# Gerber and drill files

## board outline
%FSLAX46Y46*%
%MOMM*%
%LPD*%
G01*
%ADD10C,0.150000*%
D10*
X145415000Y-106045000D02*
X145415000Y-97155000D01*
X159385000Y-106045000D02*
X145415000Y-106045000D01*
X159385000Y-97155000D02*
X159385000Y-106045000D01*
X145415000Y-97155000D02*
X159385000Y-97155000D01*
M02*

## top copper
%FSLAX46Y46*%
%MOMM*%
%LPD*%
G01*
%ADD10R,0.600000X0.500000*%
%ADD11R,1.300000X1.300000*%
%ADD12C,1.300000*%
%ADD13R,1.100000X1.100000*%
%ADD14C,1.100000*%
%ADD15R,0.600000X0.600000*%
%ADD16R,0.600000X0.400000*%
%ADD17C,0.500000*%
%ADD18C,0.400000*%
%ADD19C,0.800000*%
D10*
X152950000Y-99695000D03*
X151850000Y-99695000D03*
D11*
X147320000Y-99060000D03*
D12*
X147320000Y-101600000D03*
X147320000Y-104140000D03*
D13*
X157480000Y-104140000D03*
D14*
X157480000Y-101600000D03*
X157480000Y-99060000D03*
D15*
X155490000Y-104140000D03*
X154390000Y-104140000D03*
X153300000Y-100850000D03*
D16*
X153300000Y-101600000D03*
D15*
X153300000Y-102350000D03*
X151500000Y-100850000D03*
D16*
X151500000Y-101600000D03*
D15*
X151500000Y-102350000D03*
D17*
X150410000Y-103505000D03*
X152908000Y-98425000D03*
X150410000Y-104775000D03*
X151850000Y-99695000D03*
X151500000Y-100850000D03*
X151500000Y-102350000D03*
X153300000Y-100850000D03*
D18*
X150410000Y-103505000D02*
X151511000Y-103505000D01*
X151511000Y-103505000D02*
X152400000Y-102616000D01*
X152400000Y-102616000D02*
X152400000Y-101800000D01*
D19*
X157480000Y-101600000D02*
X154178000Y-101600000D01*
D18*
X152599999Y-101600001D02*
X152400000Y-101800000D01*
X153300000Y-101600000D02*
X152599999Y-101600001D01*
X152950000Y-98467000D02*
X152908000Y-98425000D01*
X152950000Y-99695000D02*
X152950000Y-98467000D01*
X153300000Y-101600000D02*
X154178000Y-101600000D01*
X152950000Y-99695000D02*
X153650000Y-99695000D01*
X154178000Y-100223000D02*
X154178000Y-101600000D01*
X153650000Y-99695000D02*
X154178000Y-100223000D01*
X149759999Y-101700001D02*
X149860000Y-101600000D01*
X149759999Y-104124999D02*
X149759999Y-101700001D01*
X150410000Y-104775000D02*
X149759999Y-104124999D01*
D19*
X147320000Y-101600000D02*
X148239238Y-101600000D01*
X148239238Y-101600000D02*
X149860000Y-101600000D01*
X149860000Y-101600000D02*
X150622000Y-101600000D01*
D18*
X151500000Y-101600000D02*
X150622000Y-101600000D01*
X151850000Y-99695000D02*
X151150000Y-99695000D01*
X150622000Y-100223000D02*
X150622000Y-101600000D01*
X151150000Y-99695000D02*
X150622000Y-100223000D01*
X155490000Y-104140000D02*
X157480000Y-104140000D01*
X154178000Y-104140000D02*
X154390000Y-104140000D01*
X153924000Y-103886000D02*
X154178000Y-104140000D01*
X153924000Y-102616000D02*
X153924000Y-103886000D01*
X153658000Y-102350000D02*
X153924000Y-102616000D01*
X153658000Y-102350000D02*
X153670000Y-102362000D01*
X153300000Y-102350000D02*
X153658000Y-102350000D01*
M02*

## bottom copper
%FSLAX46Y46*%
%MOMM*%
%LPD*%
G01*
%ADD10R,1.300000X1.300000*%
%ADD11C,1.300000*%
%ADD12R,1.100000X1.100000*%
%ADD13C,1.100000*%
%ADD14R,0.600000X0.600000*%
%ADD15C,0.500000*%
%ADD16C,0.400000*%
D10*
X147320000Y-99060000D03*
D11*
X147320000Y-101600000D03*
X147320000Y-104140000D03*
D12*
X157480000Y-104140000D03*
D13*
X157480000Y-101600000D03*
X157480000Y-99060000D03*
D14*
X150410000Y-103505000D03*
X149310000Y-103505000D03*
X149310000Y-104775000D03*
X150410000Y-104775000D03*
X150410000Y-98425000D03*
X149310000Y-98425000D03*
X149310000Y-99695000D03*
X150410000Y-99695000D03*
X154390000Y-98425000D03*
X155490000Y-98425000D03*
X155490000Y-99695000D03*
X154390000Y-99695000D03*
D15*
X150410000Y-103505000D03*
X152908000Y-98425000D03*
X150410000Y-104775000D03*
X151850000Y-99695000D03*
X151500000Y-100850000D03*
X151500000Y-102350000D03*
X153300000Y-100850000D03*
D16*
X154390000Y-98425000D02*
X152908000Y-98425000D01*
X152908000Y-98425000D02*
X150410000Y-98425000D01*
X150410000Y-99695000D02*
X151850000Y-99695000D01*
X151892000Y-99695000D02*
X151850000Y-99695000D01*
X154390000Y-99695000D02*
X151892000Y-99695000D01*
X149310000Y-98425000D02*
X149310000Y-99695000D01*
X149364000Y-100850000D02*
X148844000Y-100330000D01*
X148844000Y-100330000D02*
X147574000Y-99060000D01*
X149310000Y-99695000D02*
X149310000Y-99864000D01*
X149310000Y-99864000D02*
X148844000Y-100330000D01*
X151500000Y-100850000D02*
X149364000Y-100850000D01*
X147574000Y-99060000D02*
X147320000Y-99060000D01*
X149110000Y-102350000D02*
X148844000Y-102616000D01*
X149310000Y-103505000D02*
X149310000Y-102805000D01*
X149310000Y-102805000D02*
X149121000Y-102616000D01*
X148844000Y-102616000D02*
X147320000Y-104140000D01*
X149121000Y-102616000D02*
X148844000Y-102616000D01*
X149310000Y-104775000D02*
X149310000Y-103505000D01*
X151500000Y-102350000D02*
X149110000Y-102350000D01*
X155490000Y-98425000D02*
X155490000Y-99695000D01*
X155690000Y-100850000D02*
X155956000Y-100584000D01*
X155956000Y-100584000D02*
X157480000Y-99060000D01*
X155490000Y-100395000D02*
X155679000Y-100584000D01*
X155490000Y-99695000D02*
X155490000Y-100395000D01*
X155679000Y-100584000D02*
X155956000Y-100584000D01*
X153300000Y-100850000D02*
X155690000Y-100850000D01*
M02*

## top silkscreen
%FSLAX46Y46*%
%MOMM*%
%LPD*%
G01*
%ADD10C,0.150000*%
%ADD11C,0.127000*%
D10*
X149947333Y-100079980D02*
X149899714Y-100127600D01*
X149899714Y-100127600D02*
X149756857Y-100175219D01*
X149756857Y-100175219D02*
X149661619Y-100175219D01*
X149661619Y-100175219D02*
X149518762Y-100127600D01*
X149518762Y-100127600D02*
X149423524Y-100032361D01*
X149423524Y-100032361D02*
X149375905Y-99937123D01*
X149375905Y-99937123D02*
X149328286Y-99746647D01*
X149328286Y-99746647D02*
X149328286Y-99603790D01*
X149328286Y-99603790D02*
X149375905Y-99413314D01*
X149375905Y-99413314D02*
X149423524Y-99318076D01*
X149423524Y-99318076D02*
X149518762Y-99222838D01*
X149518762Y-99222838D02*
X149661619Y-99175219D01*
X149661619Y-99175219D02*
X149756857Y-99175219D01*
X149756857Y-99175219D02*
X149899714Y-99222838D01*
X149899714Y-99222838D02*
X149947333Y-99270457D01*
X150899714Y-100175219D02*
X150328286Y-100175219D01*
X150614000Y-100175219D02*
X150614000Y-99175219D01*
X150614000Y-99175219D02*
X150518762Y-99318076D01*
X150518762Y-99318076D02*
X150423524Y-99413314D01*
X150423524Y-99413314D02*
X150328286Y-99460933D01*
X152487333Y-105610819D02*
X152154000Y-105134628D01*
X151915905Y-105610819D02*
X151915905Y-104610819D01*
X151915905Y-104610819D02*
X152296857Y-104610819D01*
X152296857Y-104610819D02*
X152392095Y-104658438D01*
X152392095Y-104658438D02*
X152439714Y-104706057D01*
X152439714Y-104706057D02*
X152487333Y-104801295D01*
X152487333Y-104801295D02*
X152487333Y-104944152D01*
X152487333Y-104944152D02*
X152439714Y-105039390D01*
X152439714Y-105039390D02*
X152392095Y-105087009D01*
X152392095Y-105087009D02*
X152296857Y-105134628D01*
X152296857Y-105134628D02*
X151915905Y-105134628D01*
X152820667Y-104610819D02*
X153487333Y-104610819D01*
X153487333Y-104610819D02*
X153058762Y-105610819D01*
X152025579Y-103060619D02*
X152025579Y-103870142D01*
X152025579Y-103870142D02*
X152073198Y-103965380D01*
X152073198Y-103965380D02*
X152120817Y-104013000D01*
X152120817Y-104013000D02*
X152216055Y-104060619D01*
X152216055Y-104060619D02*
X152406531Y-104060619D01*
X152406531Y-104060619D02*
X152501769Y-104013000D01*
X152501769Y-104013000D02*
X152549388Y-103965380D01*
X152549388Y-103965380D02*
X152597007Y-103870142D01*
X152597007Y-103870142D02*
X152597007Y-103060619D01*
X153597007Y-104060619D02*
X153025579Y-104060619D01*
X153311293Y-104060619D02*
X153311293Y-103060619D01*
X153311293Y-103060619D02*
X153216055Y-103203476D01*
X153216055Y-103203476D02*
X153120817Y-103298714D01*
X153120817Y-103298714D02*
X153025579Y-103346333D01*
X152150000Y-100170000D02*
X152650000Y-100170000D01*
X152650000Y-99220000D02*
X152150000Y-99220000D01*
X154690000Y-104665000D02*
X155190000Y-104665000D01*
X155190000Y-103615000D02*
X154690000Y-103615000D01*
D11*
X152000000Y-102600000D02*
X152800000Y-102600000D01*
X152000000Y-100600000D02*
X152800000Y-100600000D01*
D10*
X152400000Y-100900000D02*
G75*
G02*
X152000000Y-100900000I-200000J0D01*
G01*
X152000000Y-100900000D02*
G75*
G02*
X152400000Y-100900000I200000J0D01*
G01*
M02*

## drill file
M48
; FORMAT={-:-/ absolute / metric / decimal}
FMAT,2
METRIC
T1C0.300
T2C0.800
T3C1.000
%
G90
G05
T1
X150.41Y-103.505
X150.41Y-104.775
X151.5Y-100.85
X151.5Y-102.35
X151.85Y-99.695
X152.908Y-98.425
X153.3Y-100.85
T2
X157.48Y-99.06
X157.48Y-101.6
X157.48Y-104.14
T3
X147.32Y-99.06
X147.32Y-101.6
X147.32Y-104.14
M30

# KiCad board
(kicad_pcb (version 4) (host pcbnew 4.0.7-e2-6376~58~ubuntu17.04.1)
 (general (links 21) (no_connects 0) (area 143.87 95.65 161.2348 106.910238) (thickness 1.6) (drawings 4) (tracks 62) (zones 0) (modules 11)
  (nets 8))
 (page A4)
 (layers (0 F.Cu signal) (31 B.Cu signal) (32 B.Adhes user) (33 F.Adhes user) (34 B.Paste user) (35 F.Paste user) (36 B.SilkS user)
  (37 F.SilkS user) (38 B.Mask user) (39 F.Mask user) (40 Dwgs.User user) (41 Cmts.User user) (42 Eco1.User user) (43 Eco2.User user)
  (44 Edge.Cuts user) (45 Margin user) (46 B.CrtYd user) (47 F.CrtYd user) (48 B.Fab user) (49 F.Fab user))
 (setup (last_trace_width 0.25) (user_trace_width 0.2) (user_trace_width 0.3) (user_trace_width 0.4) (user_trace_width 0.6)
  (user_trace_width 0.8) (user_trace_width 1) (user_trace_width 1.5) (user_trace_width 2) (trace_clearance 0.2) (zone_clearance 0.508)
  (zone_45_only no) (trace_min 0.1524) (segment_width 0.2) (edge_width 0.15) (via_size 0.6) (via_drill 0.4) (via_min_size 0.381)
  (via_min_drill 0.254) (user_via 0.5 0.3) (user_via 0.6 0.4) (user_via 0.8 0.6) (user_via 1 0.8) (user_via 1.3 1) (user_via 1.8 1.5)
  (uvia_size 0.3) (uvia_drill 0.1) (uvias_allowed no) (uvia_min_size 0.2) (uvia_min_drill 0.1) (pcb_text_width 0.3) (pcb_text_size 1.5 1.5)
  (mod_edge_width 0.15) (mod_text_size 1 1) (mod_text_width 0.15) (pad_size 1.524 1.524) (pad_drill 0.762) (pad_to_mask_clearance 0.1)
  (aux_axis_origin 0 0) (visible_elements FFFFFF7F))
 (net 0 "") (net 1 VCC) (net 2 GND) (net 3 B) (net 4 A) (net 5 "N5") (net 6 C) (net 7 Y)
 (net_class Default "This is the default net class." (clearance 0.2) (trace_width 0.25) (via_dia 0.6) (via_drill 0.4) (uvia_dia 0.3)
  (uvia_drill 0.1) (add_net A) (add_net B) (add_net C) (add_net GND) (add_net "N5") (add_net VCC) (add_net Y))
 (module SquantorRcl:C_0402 (layer F.Cu) (at 152.4 99.695 180)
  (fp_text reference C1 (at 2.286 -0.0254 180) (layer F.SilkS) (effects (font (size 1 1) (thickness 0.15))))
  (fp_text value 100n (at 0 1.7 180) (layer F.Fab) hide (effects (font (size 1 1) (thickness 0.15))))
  (fp_line (start 0.25 -0.475) (end -0.25 -0.475) (layer F.SilkS) (width 0.15))
  (fp_line (start -0.25 0.475) (end 0.25 0.475) (layer F.SilkS) (width 0.15))
  (pad 1 smd rect (at -0.55 0 180) (size 0.6 0.5) (layers F.Cu F.Paste F.Mask) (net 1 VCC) (solder_mask_margin 0.1))
  (pad 2 smd rect (at 0.55 0 180) (size 0.6 0.5) (layers F.Cu F.Paste F.Mask) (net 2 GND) (solder_mask_margin 0.1)))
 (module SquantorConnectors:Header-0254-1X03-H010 (layer B.Cu) (at 147.32 101.6 270)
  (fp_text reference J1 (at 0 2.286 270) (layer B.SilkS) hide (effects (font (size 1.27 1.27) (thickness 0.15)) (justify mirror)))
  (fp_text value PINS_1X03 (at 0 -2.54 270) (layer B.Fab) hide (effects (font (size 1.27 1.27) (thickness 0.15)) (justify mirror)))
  (pad 1 thru_hole rect (at -2.54 0 90) (size 1.3 1.3) (drill 1) (layers *.Cu *.Mask) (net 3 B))
  (pad 2 thru_hole circle (at 0 0 90) (size 1.3 1.3) (drill 1) (layers *.Cu *.Mask) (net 2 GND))
  (pad 3 thru_hole circle (at 2.54 0 90) (size 1.3 1.3) (drill 1) (layers *.Cu *.Mask) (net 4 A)))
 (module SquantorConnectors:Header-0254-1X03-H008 (layer B.Cu) (at 157.48 101.6 90)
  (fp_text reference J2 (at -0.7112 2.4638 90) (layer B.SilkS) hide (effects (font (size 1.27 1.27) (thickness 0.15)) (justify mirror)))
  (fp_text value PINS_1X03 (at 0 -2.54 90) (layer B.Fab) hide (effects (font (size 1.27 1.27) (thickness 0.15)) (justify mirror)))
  (pad 1 thru_hole rect (at -2.54 0 270) (size 1.1 1.1) (drill 0.8) (layers *.Cu *.Mask) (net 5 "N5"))
  (pad 2 thru_hole circle (at 0 0 270) (size 1.1 1.1) (drill 0.8) (layers *.Cu *.Mask) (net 1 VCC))
  (pad 3 thru_hole circle (at 2.54 0 270) (size 1.1 1.1) (drill 0.8) (layers *.Cu *.Mask) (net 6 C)))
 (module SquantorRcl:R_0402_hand (layer B.Cu) (at 149.86 103.505 180)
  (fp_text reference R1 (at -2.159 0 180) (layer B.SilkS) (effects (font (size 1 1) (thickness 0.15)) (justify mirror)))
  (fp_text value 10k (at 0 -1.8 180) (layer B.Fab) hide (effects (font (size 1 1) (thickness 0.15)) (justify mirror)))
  (pad 1 smd rect (at -0.55 0 180) (size 0.6 0.6) (layers B.Cu B.Paste B.Mask) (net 1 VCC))
  (pad 2 smd rect (at 0.55 0 180) (size 0.6 0.6) (layers B.Cu B.Paste B.Mask) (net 4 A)))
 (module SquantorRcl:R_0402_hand (layer B.Cu) (at 149.86 104.775)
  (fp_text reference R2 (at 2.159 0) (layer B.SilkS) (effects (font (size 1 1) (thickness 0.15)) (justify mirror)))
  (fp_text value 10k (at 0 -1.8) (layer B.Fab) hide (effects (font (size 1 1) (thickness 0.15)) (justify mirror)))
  (pad 1 smd rect (at -0.55 0) (size 0.6 0.6) (layers B.Cu B.Paste B.Mask) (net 4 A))
  (pad 2 smd rect (at 0.55 0) (size 0.6 0.6) (layers B.Cu B.Paste B.Mask) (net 2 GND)))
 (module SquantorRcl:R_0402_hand (layer B.Cu) (at 149.86 98.425 180)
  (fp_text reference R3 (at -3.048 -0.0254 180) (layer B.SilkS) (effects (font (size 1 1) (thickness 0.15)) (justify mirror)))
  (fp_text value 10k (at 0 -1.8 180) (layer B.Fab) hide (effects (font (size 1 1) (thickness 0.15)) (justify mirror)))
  (pad 1 smd rect (at -0.55 0 180) (size 0.6 0.6) (layers B.Cu B.Paste B.Mask) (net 1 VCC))
  (pad 2 smd rect (at 0.55 0 180) (size 0.6 0.6) (layers B.Cu B.Paste B.Mask) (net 3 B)))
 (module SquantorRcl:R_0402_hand (layer B.Cu) (at 149.86 99.695)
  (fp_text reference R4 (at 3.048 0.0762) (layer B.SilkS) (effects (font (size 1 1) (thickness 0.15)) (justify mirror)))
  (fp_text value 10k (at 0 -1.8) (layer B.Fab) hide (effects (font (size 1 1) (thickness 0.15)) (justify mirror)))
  (pad 1 smd rect (at -0.55 0) (size 0.6 0.6) (layers B.Cu B.Paste B.Mask) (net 3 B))
  (pad 2 smd rect (at 0.55 0) (size 0.6 0.6) (layers B.Cu B.Paste B.Mask) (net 2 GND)))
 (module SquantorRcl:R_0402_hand (layer B.Cu) (at 154.94 98.425)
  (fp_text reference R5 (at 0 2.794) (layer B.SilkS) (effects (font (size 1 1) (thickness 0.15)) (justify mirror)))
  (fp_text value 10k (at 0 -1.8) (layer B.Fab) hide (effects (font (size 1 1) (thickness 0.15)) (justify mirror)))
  (pad 1 smd rect (at -0.55 0) (size 0.6 0.6) (layers B.Cu B.Paste B.Mask) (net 1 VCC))
  (pad 2 smd rect (at 0.55 0) (size 0.6 0.6) (layers B.Cu B.Paste B.Mask) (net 6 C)))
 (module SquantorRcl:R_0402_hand (layer B.Cu) (at 154.94 99.695 180)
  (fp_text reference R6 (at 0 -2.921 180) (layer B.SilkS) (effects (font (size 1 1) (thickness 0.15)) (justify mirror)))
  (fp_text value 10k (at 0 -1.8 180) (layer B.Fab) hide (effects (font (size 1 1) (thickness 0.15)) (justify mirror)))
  (pad 1 smd rect (at -0.55 0 180) (size 0.6 0.6) (layers B.Cu B.Paste B.Mask) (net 6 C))
  (pad 2 smd rect (at 0.55 0 180) (size 0.6 0.6) (layers B.Cu B.Paste B.Mask) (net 2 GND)))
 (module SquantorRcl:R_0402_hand (layer F.Cu) (at 154.94 104.14 180)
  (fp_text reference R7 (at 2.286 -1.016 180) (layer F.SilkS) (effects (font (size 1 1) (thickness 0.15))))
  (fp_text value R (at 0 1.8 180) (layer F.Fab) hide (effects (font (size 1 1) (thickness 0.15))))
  (fp_line (start 0.25 -0.525) (end -0.25 -0.525) (layer F.SilkS) (width 0.15))
  (fp_line (start -0.25 0.525) (end 0.25 0.525) (layer F.SilkS) (width 0.15))
  (pad 1 smd rect (at -0.55 0 180) (size 0.6 0.6) (layers F.Cu F.Paste F.Mask) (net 5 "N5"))
  (pad 2 smd rect (at 0.55 0 180) (size 0.6 0.6) (layers F.Cu F.Paste F.Mask) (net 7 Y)))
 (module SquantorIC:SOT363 (layer F.Cu) (at 152.4 101.6 270)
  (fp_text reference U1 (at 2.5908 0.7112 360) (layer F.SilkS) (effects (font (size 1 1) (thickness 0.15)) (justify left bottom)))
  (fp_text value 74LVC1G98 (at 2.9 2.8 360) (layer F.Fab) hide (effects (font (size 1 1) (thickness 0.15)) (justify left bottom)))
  (fp_line (start 1 0.4) (end 1 -0.4) (layer F.SilkS) (width 0.127))
  (fp_line (start -1 0.4) (end -1 -0.4) (layer F.SilkS) (width 0.127))
  (fp_circle (center -0.7 0.2) (end -0.5 0.2) (layer F.SilkS) (width 0.15))
  (pad 6 smd rect (at -0.75 -0.9 270) (size 0.6 0.6) (layers F.Cu F.Paste F.Mask) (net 6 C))
  (pad 5 smd rect (at 0 -0.9 270) (size 0.4 0.6) (layers F.Cu F.Paste F.Mask) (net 1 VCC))
  (pad 4 smd rect (at 0.75 -0.9 270) (size 0.6 0.6) (layers F.Cu F.Paste F.Mask) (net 7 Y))
  (pad 1 smd rect (at -0.75 0.9 270) (size 0.6 0.6) (layers F.Cu F.Paste F.Mask) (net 3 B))
  (pad 2 smd rect (at 0 0.9 270) (size 0.4 0.6) (layers F.Cu F.Paste F.Mask) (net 2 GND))
  (pad 3 smd rect (at 0.75 0.9 270) (size 0.6 0.6) (layers F.Cu F.Paste F.Mask) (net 4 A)))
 (gr_line (start 145.415 106.045) (end 145.415 97.155) (angle 90) (layer Edge.Cuts) (width 0.15))
 (gr_line (start 159.385 106.045) (end 145.415 106.045) (angle 90) (layer Edge.Cuts) (width 0.15))
 (gr_line (start 159.385 97.155) (end 159.385 106.045) (angle 90) (layer Edge.Cuts) (width 0.15))
 (gr_line (start 145.415 97.155) (end 159.385 97.155) (angle 90) (layer Edge.Cuts) (width 0.15))
 (segment (start 150.41 103.505) (end 151.511 103.505) (width 0.4) (layer F.Cu) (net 1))
 (segment (start 151.511 103.505) (end 152.4 102.616) (width 0.4) (layer F.Cu) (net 1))
 (segment (start 152.4 102.616) (end 152.4 101.8) (width 0.4) (layer F.Cu) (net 1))
 (via (at 150.41 103.505) (size 0.5) (drill 0.3) (layers F.Cu B.Cu) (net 1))
 (segment (start 157.48 101.6) (end 154.178 101.6) (width 0.8) (layer F.Cu) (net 1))
 (segment (start 152.599999 101.600001) (end 152.4 101.8) (width 0.4) (layer F.Cu) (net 1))
 (segment (start 153.3 101.6) (end 152.599999 101.600001) (width 0.4) (layer F.Cu) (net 1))
 (segment (start 154.39 98.425) (end 152.908 98.425) (width 0.4) (layer B.Cu) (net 1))
 (segment (start 152.908 98.425) (end 150.41 98.425) (width 0.4) (layer B.Cu) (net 1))
 (segment (start 152.95 98.467) (end 152.908 98.425) (width 0.4) (layer F.Cu) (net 1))
 (via (at 152.908 98.425) (size 0.5) (drill 0.3) (layers F.Cu B.Cu) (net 1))
 (segment (start 152.95 99.695) (end 152.95 98.467) (width 0.4) (layer F.Cu) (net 1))
 (segment (start 153.3 101.6) (end 154.178 101.6) (width 0.4) (layer F.Cu) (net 1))
 (segment (start 152.95 99.695) (end 153.65 99.695) (width 0.4) (layer F.Cu) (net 1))
 (segment (start 154.178 100.223) (end 154.178 101.6) (width 0.4) (layer F.Cu) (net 1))
 (segment (start 153.65 99.695) (end 154.178 100.223) (width 0.4) (layer F.Cu) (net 1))
 (segment (start 149.759999 101.700001) (end 149.86 101.6) (width 0.4) (layer F.Cu) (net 2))
 (segment (start 149.759999 104.124999) (end 149.759999 101.700001) (width 0.4) (layer F.Cu) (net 2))
 (segment (start 150.41 104.775) (end 149.759999 104.124999) (width 0.4) (layer F.Cu) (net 2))
 (segment (start 147.32 101.6) (end 148.239238 101.6) (width 0.8) (layer F.Cu) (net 2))
 (segment (start 148.239238 101.6) (end 149.86 101.6) (width 0.8) (layer F.Cu) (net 2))
 (segment (start 149.86 101.6) (end 150.622 101.6) (width 0.8) (layer F.Cu) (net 2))
 (via (at 150.41 104.775) (size 0.5) (drill 0.3) (layers F.Cu B.Cu) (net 2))
 (segment (start 150.41 99.695) (end 151.85 99.695) (width 0.4) (layer B.Cu) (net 2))
 (segment (start 151.892 99.695) (end 151.85 99.695) (width 0.4) (layer B.Cu) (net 2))
 (via (at 151.85 99.695) (size 0.5) (drill 0.3) (layers F.Cu B.Cu) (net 2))
 (segment (start 154.39 99.695) (end 151.892 99.695) (width 0.4) (layer B.Cu) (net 2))
 (segment (start 151.5 101.6) (end 150.622 101.6) (width 0.4) (layer F.Cu) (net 2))
 (segment (start 151.85 99.695) (end 151.15 99.695) (width 0.4) (layer F.Cu) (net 2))
 (segment (start 150.622 100.223) (end 150.622 101.6) (width 0.4) (layer F.Cu) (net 2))
 (segment (start 151.15 99.695) (end 150.622 100.223) (width 0.4) (layer F.Cu) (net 2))
 (segment (start 149.31 98.425) (end 149.31 99.695) (width 0.4) (layer B.Cu) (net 3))
 (segment (start 149.364 100.85) (end 148.844 100.33) (width 0.4) (layer B.Cu) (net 3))
 (segment (start 148.844 100.33) (end 147.574 99.06) (width 0.4) (layer B.Cu) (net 3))
 (segment (start 149.31 99.695) (end 149.31 99.864) (width 0.4) (layer B.Cu) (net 3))
 (segment (start 149.31 99.864) (end 148.844 100.33) (width 0.4) (layer B.Cu) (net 3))
 (segment (start 151.5 100.85) (end 149.364 100.85) (width 0.4) (layer B.Cu) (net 3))
 (segment (start 147.574 99.06) (end 147.32 99.06) (width 0.4) (layer B.Cu) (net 3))
 (via (at 151.5 100.85) (size 0.5) (drill 0.3) (layers F.Cu B.Cu) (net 3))
 (segment (start 149.11 102.35) (end 148.844 102.616) (width 0.4) (layer B.Cu) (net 4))
 (segment (start 149.31 103.505) (end 149.31 102.805) (width 0.4) (layer B.Cu) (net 4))
 (segment (start 149.31 102.805) (end 149.121 102.616) (width 0.4) (layer B.Cu) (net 4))
 (segment (start 148.844 102.616) (end 147.32 104.14) (width 0.4) (layer B.Cu) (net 4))
 (segment (start 149.121 102.616) (end 148.844 102.616) (width 0.4) (layer B.Cu) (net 4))
 (segment (start 149.31 104.775) (end 149.31 103.505) (width 0.4) (layer B.Cu) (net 4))
 (segment (start 151.5 102.35) (end 149.11 102.35) (width 0.4) (layer B.Cu) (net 4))
 (via (at 151.5 102.35) (size 0.5) (drill 0.3) (layers F.Cu B.Cu) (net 4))
 (segment (start 155.49 104.14) (end 157.48 104.14) (width 0.4) (layer F.Cu) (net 5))
 (segment (start 155.49 98.425) (end 155.49 99.695) (width 0.4) (layer B.Cu) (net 6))
 (segment (start 155.69 100.85) (end 155.956 100.584) (width 0.4) (layer B.Cu) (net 6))
 (segment (start 155.956 100.584) (end 157.48 99.06) (width 0.4) (layer B.Cu) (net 6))
 (segment (start 155.49 100.395) (end 155.679 100.584) (width 0.4) (layer B.Cu) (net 6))
 (segment (start 155.49 99.695) (end 155.49 100.395) (width 0.4) (layer B.Cu) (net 6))
 (segment (start 155.679 100.584) (end 155.956 100.584) (width 0.4) (layer B.Cu) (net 6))
 (segment (start 153.3 100.85) (end 155.69 100.85) (width 0.4) (layer B.Cu) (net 6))
 (via (at 153.3 100.85) (size 0.5) (drill 0.3) (layers F.Cu B.Cu) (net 6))
 (segment (start 154.178 104.14) (end 154.39 104.14) (width 0.4) (layer F.Cu) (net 7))
 (segment (start 153.924 103.886) (end 154.178 104.14) (width 0.4) (layer F.Cu) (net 7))
 (segment (start 153.924 102.616) (end 153.924 103.886) (width 0.4) (layer F.Cu) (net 7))
 (segment (start 153.658 102.35) (end 153.924 102.616) (width 0.4) (layer F.Cu) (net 7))
 (segment (start 153.658 102.35) (end 153.67 102.362) (width 0.4) (layer F.Cu) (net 7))
 (segment (start 153.3 102.35) (end 153.658 102.35) (width 0.4) (layer F.Cu) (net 7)))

